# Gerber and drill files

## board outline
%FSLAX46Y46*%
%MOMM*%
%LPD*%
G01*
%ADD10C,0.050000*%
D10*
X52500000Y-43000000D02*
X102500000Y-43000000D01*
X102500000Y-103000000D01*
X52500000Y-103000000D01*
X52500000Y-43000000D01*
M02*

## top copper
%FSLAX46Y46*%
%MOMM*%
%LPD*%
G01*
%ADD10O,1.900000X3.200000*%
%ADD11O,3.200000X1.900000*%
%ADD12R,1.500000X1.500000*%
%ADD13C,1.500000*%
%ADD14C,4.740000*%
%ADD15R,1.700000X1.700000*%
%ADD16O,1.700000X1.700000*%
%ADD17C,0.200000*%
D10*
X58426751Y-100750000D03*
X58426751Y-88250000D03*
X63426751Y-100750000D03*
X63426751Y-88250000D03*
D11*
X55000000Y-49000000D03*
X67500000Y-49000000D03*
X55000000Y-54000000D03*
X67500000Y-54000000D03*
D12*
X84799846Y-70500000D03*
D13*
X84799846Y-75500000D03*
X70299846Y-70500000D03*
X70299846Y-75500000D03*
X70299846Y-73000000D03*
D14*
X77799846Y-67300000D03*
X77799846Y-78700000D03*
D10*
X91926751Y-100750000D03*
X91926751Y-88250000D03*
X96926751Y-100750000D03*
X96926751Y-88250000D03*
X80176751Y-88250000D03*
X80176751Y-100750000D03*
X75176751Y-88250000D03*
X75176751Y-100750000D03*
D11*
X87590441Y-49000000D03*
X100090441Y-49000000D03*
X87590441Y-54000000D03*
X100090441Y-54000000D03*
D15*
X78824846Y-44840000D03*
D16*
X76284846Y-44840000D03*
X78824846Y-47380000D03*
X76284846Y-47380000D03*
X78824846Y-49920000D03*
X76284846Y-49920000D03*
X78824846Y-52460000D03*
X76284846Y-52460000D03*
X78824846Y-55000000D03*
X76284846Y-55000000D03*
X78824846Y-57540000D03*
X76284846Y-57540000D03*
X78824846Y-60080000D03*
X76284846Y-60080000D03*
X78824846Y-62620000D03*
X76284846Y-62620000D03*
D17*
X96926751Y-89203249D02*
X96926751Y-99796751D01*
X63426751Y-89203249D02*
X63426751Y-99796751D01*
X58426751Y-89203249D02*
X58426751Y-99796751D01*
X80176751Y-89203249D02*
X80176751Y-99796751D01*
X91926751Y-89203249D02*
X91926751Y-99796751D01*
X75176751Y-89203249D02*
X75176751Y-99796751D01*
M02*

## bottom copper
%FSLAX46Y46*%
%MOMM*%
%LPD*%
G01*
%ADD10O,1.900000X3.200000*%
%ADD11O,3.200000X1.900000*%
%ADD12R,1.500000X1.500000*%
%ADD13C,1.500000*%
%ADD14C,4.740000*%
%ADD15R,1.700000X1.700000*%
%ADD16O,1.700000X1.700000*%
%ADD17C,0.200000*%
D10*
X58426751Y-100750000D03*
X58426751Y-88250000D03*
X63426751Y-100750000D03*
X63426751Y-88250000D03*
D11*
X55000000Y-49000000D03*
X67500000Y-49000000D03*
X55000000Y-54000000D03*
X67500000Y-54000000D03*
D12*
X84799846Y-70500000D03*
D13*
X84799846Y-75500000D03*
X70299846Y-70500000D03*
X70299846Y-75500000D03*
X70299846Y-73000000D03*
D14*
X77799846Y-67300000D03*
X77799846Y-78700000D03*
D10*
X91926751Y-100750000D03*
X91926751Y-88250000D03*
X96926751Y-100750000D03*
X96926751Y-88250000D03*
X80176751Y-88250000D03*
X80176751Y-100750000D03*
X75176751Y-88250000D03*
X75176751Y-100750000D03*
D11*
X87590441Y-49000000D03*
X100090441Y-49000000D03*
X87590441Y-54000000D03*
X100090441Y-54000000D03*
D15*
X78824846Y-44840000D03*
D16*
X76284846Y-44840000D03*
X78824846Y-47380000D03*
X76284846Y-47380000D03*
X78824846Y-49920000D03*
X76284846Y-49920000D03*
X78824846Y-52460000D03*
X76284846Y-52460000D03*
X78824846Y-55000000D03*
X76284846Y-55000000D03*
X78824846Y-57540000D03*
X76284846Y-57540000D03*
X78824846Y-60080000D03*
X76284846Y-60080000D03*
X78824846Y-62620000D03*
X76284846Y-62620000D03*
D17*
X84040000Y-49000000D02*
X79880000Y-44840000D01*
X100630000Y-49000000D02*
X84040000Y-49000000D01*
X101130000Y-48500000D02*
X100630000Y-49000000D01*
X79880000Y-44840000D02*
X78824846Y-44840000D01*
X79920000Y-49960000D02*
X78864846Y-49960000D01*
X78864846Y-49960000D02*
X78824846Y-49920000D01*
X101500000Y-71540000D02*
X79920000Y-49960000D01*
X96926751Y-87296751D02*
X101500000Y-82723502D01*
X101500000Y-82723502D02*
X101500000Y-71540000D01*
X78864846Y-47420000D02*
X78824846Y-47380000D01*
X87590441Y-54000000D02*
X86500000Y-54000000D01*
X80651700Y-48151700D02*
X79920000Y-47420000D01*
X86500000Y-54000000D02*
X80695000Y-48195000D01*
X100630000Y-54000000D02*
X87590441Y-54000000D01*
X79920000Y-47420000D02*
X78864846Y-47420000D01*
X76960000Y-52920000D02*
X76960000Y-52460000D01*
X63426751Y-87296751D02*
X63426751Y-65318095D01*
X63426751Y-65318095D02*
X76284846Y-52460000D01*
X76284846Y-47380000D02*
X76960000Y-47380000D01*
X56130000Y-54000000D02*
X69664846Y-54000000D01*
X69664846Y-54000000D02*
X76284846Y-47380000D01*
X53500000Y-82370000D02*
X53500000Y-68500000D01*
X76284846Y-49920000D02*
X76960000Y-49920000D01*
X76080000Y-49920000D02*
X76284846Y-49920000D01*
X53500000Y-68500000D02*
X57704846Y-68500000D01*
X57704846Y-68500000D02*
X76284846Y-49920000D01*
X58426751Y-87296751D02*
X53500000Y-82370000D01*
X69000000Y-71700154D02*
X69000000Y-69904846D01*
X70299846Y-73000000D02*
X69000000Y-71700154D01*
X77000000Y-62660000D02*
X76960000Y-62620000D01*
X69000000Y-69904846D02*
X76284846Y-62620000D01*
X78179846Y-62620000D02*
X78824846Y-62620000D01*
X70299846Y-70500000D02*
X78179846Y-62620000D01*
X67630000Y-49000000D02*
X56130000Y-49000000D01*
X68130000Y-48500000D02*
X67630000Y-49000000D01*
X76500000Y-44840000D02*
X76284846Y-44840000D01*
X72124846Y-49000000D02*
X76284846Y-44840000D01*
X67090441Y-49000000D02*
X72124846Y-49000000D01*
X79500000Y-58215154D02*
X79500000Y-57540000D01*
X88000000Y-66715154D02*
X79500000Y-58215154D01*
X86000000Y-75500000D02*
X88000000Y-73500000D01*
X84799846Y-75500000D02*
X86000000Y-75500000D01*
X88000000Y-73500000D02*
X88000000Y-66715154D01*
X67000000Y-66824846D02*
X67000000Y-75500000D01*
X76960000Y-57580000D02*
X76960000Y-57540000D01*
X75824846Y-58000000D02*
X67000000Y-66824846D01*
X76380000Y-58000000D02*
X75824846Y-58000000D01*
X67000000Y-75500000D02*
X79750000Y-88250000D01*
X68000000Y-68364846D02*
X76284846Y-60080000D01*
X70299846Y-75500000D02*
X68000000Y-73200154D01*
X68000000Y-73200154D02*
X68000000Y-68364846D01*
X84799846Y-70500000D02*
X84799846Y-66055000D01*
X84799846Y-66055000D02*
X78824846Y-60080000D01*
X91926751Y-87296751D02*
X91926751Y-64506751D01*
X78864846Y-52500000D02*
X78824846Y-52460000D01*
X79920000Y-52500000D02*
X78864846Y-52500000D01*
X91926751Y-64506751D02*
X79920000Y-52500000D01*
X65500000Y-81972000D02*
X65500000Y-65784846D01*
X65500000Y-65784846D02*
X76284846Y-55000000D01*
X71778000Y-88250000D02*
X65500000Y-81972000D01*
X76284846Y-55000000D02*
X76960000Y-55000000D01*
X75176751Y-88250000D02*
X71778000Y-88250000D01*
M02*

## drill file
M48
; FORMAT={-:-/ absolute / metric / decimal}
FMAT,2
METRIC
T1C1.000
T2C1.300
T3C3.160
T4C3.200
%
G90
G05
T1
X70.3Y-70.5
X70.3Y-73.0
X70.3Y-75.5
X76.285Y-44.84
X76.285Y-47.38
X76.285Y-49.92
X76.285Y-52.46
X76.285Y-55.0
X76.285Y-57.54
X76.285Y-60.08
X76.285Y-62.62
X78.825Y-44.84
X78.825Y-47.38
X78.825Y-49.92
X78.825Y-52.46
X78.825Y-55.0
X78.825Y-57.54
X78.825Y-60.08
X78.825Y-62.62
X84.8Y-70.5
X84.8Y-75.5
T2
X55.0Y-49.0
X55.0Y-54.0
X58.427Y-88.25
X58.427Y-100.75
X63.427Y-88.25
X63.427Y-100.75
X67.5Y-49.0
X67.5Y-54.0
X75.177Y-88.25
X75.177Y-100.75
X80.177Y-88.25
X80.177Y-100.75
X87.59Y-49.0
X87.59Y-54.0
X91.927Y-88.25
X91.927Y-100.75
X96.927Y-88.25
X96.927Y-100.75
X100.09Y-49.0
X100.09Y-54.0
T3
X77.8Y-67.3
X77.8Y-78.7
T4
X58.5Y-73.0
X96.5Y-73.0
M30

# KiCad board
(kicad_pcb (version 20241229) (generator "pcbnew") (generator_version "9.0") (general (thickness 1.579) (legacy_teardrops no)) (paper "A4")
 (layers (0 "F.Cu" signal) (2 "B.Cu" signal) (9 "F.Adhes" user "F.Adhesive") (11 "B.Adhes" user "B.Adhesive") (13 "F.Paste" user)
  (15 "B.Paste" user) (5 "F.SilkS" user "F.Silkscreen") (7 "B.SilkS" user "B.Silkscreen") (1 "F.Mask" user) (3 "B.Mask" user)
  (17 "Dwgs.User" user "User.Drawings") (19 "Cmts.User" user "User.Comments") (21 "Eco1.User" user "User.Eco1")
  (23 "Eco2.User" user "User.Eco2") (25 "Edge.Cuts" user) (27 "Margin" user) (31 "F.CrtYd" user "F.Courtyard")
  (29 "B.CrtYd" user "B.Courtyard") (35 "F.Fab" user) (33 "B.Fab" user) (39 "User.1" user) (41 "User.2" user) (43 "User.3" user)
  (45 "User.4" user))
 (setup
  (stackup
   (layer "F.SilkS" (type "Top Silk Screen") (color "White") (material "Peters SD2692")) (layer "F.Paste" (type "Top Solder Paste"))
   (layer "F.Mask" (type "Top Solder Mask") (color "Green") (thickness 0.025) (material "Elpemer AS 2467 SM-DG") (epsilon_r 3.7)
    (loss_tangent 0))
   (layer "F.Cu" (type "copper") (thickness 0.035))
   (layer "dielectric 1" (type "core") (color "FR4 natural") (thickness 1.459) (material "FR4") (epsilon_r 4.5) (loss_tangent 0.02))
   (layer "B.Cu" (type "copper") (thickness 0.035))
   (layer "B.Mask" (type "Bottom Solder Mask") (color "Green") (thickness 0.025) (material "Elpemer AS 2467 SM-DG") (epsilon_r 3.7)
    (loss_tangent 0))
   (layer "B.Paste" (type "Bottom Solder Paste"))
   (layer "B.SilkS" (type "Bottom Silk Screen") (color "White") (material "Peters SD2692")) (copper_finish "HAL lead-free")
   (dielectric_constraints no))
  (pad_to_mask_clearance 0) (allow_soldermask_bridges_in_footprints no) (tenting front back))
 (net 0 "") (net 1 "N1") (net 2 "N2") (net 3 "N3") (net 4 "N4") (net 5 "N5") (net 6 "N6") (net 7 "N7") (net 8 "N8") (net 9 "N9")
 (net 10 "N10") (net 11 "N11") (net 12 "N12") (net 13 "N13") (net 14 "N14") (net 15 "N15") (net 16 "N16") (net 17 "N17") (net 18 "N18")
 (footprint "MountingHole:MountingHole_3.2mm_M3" (layer "F.Cu") (at 58.5 73)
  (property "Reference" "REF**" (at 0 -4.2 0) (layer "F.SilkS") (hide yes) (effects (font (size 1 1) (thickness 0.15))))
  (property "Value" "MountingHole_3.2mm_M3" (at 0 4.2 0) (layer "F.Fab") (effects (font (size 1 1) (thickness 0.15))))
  (pad "" np_thru_hole circle (at 0 0) (size 3.2 3.2) (drill 3.2) (layers "*.Cu" "*.Mask")))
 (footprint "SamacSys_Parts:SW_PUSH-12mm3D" (layer "F.Cu") (at 58.426751 100.75 90)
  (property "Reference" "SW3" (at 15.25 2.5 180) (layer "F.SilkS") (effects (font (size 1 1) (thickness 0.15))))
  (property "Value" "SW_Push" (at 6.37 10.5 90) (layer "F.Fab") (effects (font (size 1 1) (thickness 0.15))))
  (pad "1" thru_hole oval (at 0 0 90) (size 3.2 1.9) (drill 1.3) (layers "*.Cu" "*.Mask") (remove_unused_layers no) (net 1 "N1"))
  (pad "1" thru_hole oval (at 12.5 0 90) (size 3.2 1.9) (drill 1.3) (layers "*.Cu" "*.Mask") (remove_unused_layers no) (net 1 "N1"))
  (pad "2" thru_hole oval (at 0 5 90) (size 3.2 1.9) (drill 1.3) (layers "*.Cu" "*.Mask") (remove_unused_layers no) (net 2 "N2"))
  (pad "2" thru_hole oval (at 12.5 5 90) (size 3.2 1.9) (drill 1.3) (layers "*.Cu" "*.Mask") (remove_unused_layers no) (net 2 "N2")))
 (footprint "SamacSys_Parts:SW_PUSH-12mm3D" (layer "F.Cu") (at 55 49)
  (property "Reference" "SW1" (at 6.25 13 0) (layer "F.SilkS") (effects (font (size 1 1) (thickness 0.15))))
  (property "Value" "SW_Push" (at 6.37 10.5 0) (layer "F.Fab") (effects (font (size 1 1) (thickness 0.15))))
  (pad "1" thru_hole oval (at 0 0) (size 3.2 1.9) (drill 1.3) (layers "*.Cu" "*.Mask") (remove_unused_layers no) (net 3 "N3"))
  (pad "1" thru_hole oval (at 12.5 0) (size 3.2 1.9) (drill 1.3) (layers "*.Cu" "*.Mask") (remove_unused_layers no) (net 3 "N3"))
  (pad "2" thru_hole oval (at 0 5) (size 3.2 1.9) (drill 1.3) (layers "*.Cu" "*.Mask") (remove_unused_layers no) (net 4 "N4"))
  (pad "2" thru_hole oval (at 12.5 5) (size 3.2 1.9) (drill 1.3) (layers "*.Cu" "*.Mask") (remove_unused_layers no) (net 4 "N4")))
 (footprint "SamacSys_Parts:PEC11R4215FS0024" (layer "F.Cu") (at 84.799846 70.5 -90)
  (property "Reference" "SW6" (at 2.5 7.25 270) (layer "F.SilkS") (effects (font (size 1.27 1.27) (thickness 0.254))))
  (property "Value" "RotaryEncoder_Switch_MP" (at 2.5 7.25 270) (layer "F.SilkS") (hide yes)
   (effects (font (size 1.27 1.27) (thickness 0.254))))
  (pad "1" thru_hole rect (at 0 0 270) (size 1.5 1.5) (drill 1) (layers "*.Cu" "*.Mask") (remove_unused_layers no) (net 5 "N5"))
  (pad "2" thru_hole circle (at 5 0 270) (size 1.5 1.5) (drill 1) (layers "*.Cu" "*.Mask") (remove_unused_layers no) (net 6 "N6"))
  (pad "A1" thru_hole circle (at 0 14.5 270) (size 1.5 1.5) (drill 1) (layers "*.Cu" "*.Mask") (remove_unused_layers no) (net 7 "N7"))
  (pad "B1" thru_hole circle (at 5 14.5 270) (size 1.5 1.5) (drill 1) (layers "*.Cu" "*.Mask") (remove_unused_layers no) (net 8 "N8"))
  (pad "C1" thru_hole circle (at 2.5 14.5 270) (size 1.5 1.5) (drill 1) (layers "*.Cu" "*.Mask") (remove_unused_layers no) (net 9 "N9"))
  (pad "MH1" thru_hole circle (at -3.2 7 270) (size 4.74 4.74) (drill 3.16) (layers "*.Cu" "*.Mask") (remove_unused_layers no)
   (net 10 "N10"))
  (pad "MH2" thru_hole circle (at 8.2 7 270) (size 4.74 4.74) (drill 3.16) (layers "*.Cu" "*.Mask") (remove_unused_layers no) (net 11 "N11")))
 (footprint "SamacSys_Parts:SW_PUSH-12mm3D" (layer "F.Cu") (at 91.926751 100.75 90)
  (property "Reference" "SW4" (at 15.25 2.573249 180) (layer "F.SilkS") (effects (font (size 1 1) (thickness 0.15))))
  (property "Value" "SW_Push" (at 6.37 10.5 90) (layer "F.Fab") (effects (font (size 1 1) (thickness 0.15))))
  (pad "1" thru_hole oval (at 0 0 90) (size 3.2 1.9) (drill 1.3) (layers "*.Cu" "*.Mask") (remove_unused_layers no) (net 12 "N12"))
  (pad "1" thru_hole oval (at 12.5 0 90) (size 3.2 1.9) (drill 1.3) (layers "*.Cu" "*.Mask") (remove_unused_layers no) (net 12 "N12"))
  (pad "2" thru_hole oval (at 0 5 90) (size 3.2 1.9) (drill 1.3) (layers "*.Cu" "*.Mask") (remove_unused_layers no) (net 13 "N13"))
  (pad "2" thru_hole oval (at 12.5 5 90) (size 3.2 1.9) (drill 1.3) (layers "*.Cu" "*.Mask") (remove_unused_layers no) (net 13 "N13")))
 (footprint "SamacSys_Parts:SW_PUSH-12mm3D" (layer "F.Cu") (at 80.176751 88.25 -90)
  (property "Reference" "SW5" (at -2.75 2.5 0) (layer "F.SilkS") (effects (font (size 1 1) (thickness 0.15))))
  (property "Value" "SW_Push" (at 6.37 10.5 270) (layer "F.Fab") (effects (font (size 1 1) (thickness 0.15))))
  (pad "1" thru_hole oval (at 0 0 270) (size 3.2 1.9) (drill 1.3) (layers "*.Cu" "*.Mask") (remove_unused_layers no) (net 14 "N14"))
  (pad "1" thru_hole oval (at 12.5 0 270) (size 3.2 1.9) (drill 1.3) (layers "*.Cu" "*.Mask") (remove_unused_layers no) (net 14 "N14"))
  (pad "2" thru_hole oval (at 0 5 270) (size 3.2 1.9) (drill 1.3) (layers "*.Cu" "*.Mask") (remove_unused_layers no) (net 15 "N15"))
  (pad "2" thru_hole oval (at 12.5 5 270) (size 3.2 1.9) (drill 1.3) (layers "*.Cu" "*.Mask") (remove_unused_layers no) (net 15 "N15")))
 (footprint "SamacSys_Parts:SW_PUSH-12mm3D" (layer "F.Cu") (at 87.590441 49)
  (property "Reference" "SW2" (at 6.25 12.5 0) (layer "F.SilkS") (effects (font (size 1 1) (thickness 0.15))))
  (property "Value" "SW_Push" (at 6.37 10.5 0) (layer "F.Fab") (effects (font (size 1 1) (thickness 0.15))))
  (pad "1" thru_hole oval (at 0 0) (size 3.2 1.9) (drill 1.3) (layers "*.Cu" "*.Mask") (remove_unused_layers no) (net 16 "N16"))
  (pad "1" thru_hole oval (at 12.5 0) (size 3.2 1.9) (drill 1.3) (layers "*.Cu" "*.Mask") (remove_unused_layers no) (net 16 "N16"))
  (pad "2" thru_hole oval (at 0 5) (size 3.2 1.9) (drill 1.3) (layers "*.Cu" "*.Mask") (remove_unused_layers no) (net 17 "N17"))
  (pad "2" thru_hole oval (at 12.5 5) (size 3.2 1.9) (drill 1.3) (layers "*.Cu" "*.Mask") (remove_unused_layers no) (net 17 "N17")))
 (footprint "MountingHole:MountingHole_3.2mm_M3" (layer "F.Cu") (at 96.5 73)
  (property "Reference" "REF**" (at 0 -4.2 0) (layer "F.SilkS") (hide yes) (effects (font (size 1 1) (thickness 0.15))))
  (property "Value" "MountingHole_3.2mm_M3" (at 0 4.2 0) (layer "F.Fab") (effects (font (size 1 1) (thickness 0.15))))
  (pad "" np_thru_hole circle (at 0 0) (size 3.2 3.2) (drill 3.2) (layers "*.Cu" "*.Mask")))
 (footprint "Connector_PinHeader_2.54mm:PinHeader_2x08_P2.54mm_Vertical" (layer "B.Cu") (at 78.824846 44.84 180)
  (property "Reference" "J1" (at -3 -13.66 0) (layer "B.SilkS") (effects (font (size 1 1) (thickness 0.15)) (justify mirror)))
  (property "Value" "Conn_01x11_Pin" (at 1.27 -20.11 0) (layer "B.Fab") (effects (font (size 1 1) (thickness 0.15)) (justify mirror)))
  (pad "1" thru_hole rect (at 0 0 180) (size 1.7 1.7) (drill 1) (layers "*.Cu" "*.Mask") (remove_unused_layers no) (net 16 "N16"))
  (pad "2" thru_hole oval (at 2.54 0 180) (size 1.7 1.7) (drill 1) (layers "*.Cu" "*.Mask") (remove_unused_layers no) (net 3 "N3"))
  (pad "3" thru_hole oval (at 0 -2.54 180) (size 1.7 1.7) (drill 1) (layers "*.Cu" "*.Mask") (remove_unused_layers no) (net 17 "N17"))
  (pad "4" thru_hole oval (at 2.54 -2.54 180) (size 1.7 1.7) (drill 1) (layers "*.Cu" "*.Mask") (remove_unused_layers no) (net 4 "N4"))
  (pad "5" thru_hole oval (at 0 -5.08 180) (size 1.7 1.7) (drill 1) (layers "*.Cu" "*.Mask") (remove_unused_layers no) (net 13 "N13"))
  (pad "6" thru_hole oval (at 2.54 -5.08 180) (size 1.7 1.7) (drill 1) (layers "*.Cu" "*.Mask") (remove_unused_layers no) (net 1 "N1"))
  (pad "7" thru_hole oval (at 0 -7.62 180) (size 1.7 1.7) (drill 1) (layers "*.Cu" "*.Mask") (remove_unused_layers no) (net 12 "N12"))
  (pad "8" thru_hole oval (at 2.54 -7.62 180) (size 1.7 1.7) (drill 1) (layers "*.Cu" "*.Mask") (remove_unused_layers no) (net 2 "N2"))
  (pad "9" thru_hole oval (at 0 -10.16 180) (size 1.7 1.7) (drill 1) (layers "*.Cu" "*.Mask") (remove_unused_layers no) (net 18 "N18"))
  (pad "10" thru_hole oval (at 2.54 -10.16 180) (size 1.7 1.7) (drill 1) (layers "*.Cu" "*.Mask") (remove_unused_layers no) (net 15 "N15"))
  (pad "11" thru_hole oval (at 0 -12.7 180) (size 1.7 1.7) (drill 1) (layers "*.Cu" "*.Mask") (remove_unused_layers no) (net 6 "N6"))
  (pad "12" thru_hole oval (at 2.54 -12.7 180) (size 1.7 1.7) (drill 1) (layers "*.Cu" "*.Mask") (remove_unused_layers no) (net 14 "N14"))
  (pad "13" thru_hole oval (at 0 -15.24 180) (size 1.7 1.7) (drill 1) (layers "*.Cu" "*.Mask") (remove_unused_layers no) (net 5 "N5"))
  (pad "14" thru_hole oval (at 2.54 -15.24 180) (size 1.7 1.7) (drill 1) (layers "*.Cu" "*.Mask") (remove_unused_layers no) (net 8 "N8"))
  (pad "15" thru_hole oval (at 0 -17.78 180) (size 1.7 1.7) (drill 1) (layers "*.Cu" "*.Mask") (remove_unused_layers no) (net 7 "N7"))
  (pad "16" thru_hole oval (at 2.54 -17.78 180) (size 1.7 1.7) (drill 1) (layers "*.Cu" "*.Mask") (remove_unused_layers no) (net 9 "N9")))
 (gr_rect (start 52.5 43) (end 102.5 103) (stroke (width 0.05) (type default)) (fill no) (layer "Edge.Cuts"))
 (segment (start 84.04 49) (end 79.88 44.84) (width 0.2) (layer "B.Cu") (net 16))
 (segment (start 100.63 49) (end 84.04 49) (width 0.2) (layer "B.Cu") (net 16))
 (segment (start 101.13 48.5) (end 100.63 49) (width 0.2) (layer "B.Cu") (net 16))
 (segment (start 79.88 44.84) (end 78.824846 44.84) (width 0.2) (layer "B.Cu") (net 16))
 (segment (start 96.926751 89.203249) (end 96.926751 99.796751) (width 0.2) (layer "F.Cu") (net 13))
 (segment (start 79.92 49.96) (end 78.864846 49.96) (width 0.2) (layer "B.Cu") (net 13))
 (segment (start 78.864846 49.96) (end 78.824846 49.92) (width 0.2) (layer "B.Cu") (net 13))
 (segment (start 101.5 71.54) (end 79.92 49.96) (width 0.2) (layer "B.Cu") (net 13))
 (segment (start 96.926751 87.296751) (end 101.5 82.723502) (width 0.2) (layer "B.Cu") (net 13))
 (segment (start 101.5 82.723502) (end 101.5 71.54) (width 0.2) (layer "B.Cu") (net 13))
 (segment (start 78.864846 47.42) (end 78.824846 47.38) (width 0.2) (layer "B.Cu") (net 17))
 (segment (start 87.590441 54) (end 86.5 54) (width 0.2) (layer "B.Cu") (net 17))
 (segment (start 80.6517 48.1517) (end 79.92 47.42) (width 0.2) (layer "B.Cu") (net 17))
 (segment (start 86.5 54) (end 80.695 48.195) (width 0.2) (layer "B.Cu") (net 17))
 (segment (start 100.63 54) (end 87.590441 54) (width 0.2) (layer "B.Cu") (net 17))
 (segment (start 79.92 47.42) (end 78.864846 47.42) (width 0.2) (layer "B.Cu") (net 17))
 (segment (start 63.426751 89.203249) (end 63.426751 99.796751) (width 0.2) (layer "F.Cu") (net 2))
 (segment (start 76.96 52.92) (end 76.96 52.46) (width 0.2) (layer "B.Cu") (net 2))
 (segment (start 63.426751 87.296751) (end 63.426751 65.318095) (width 0.2) (layer "B.Cu") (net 2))
 (segment (start 63.426751 65.318095) (end 76.284846 52.46) (width 0.2) (layer "B.Cu") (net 2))
 (segment (start 76.284846 47.38) (end 76.96 47.38) (width 0.2) (layer "B.Cu") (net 4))
 (segment (start 56.13 54) (end 69.664846 54) (width 0.2) (layer "B.Cu") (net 4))
 (segment (start 69.664846 54) (end 76.284846 47.38) (width 0.2) (layer "B.Cu") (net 4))
 (segment (start 58.426751 89.203249) (end 58.426751 99.796751) (width 0.2) (layer "F.Cu") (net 1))
 (segment (start 53.5 82.37) (end 53.5 68.5) (width 0.2) (layer "B.Cu") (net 1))
 (segment (start 76.284846 49.92) (end 76.96 49.92) (width 0.2) (layer "B.Cu") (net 1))
 (segment (start 76.08 49.92) (end 76.284846 49.92) (width 0.2) (layer "B.Cu") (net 1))
 (segment (start 53.5 68.5) (end 57.704846 68.5) (width 0.2) (layer "B.Cu") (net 1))
 (segment (start 57.704846 68.5) (end 76.284846 49.92) (width 0.2) (layer "B.Cu") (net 1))
 (segment (start 58.426751 87.296751) (end 53.5 82.37) (width 0.2) (layer "B.Cu") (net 1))
 (segment (start 69 71.700154) (end 69 69.904846) (width 0.2) (layer "B.Cu") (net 9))
 (segment (start 70.299846 73) (end 69 71.700154) (width 0.2) (layer "B.Cu") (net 9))
 (segment (start 77 62.66) (end 76.96 62.62) (width 0.2) (layer "B.Cu") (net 9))
 (segment (start 69 69.904846) (end 76.284846 62.62) (width 0.2) (layer "B.Cu") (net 9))
 (segment (start 78.179846 62.62) (end 78.824846 62.62) (width 0.2) (layer "B.Cu") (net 7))
 (segment (start 70.299846 70.5) (end 78.179846 62.62) (width 0.2) (layer "B.Cu") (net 7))
 (segment (start 67.63 49) (end 56.13 49) (width 0.2) (layer "B.Cu") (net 3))
 (segment (start 68.13 48.5) (end 67.63 49) (width 0.2) (layer "B.Cu") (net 3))
 (segment (start 76.5 44.84) (end 76.284846 44.84) (width 0.2) (layer "B.Cu") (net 3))
 (segment (start 72.124846 49) (end 76.284846 44.84) (width 0.2) (layer "B.Cu") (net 3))
 (segment (start 67.090441 49) (end 72.124846 49) (width 0.2) (layer "B.Cu") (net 3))
 (segment (start 79.5 58.215154) (end 79.5 57.54) (width 0.2) (layer "B.Cu") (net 6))
 (segment (start 88 66.715154) (end 79.5 58.215154) (width 0.2) (layer "B.Cu") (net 6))
 (segment (start 86 75.5) (end 88 73.5) (width 0.2) (layer "B.Cu") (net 6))
 (segment (start 84.799846 75.5) (end 86 75.5) (width 0.2) (layer "B.Cu") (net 6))
 (segment (start 88 73.5) (end 88 66.715154) (width 0.2) (layer "B.Cu") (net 6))
 (segment (start 80.176751 89.203249) (end 80.176751 99.796751) (width 0.2) (layer "F.Cu") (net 14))
 (segment (start 67 66.824846) (end 67 75.5) (width 0.2) (layer "B.Cu") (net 14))
 (segment (start 76.96 57.58) (end 76.96 57.54) (width 0.2) (layer "B.Cu") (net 14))
 (segment (start 75.824846 58) (end 67 66.824846) (width 0.2) (layer "B.Cu") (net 14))
 (segment (start 76.38 58) (end 75.824846 58) (width 0.2) (layer "B.Cu") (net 14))
 (segment (start 67 75.5) (end 79.75 88.25) (width 0.2) (layer "B.Cu") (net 14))
 (segment (start 68 68.364846) (end 76.284846 60.08) (width 0.2) (layer "B.Cu") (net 8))
 (segment (start 70.299846 75.5) (end 68 73.200154) (width 0.2) (layer "B.Cu") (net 8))
 (segment (start 68 73.200154) (end 68 68.364846) (width 0.2) (layer "B.Cu") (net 8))
 (segment (start 84.799846 70.5) (end 84.799846 66.055) (width 0.2) (layer "B.Cu") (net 5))
 (segment (start 84.799846 66.055) (end 78.824846 60.08) (width 0.2) (layer "B.Cu") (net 5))
 (segment (start 91.926751 89.203249) (end 91.926751 99.796751) (width 0.2) (layer "F.Cu") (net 12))
 (segment (start 91.926751 87.296751) (end 91.926751 64.506751) (width 0.2) (layer "B.Cu") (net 12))
 (segment (start 78.864846 52.5) (end 78.824846 52.46) (width 0.2) (layer "B.Cu") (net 12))
 (segment (start 79.92 52.5) (end 78.864846 52.5) (width 0.2) (layer "B.Cu") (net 12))
 (segment (start 91.926751 64.506751) (end 79.92 52.5) (width 0.2) (layer "B.Cu") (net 12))
 (segment (start 75.176751 89.203249) (end 75.176751 99.796751) (width 0.2) (layer "F.Cu") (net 15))
 (segment (start 65.5 81.972) (end 65.5 65.784846) (width 0.2) (layer "B.Cu") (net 15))
 (segment (start 65.5 65.784846) (end 76.284846 55) (width 0.2) (layer "B.Cu") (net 15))
 (segment (start 71.778 88.25) (end 65.5 81.972) (width 0.2) (layer "B.Cu") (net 15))
 (segment (start 76.284846 55) (end 76.96 55) (width 0.2) (layer "B.Cu") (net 15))
 (segment (start 75.176751 88.25) (end 71.778 88.25) (width 0.2) (layer "B.Cu") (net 15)))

